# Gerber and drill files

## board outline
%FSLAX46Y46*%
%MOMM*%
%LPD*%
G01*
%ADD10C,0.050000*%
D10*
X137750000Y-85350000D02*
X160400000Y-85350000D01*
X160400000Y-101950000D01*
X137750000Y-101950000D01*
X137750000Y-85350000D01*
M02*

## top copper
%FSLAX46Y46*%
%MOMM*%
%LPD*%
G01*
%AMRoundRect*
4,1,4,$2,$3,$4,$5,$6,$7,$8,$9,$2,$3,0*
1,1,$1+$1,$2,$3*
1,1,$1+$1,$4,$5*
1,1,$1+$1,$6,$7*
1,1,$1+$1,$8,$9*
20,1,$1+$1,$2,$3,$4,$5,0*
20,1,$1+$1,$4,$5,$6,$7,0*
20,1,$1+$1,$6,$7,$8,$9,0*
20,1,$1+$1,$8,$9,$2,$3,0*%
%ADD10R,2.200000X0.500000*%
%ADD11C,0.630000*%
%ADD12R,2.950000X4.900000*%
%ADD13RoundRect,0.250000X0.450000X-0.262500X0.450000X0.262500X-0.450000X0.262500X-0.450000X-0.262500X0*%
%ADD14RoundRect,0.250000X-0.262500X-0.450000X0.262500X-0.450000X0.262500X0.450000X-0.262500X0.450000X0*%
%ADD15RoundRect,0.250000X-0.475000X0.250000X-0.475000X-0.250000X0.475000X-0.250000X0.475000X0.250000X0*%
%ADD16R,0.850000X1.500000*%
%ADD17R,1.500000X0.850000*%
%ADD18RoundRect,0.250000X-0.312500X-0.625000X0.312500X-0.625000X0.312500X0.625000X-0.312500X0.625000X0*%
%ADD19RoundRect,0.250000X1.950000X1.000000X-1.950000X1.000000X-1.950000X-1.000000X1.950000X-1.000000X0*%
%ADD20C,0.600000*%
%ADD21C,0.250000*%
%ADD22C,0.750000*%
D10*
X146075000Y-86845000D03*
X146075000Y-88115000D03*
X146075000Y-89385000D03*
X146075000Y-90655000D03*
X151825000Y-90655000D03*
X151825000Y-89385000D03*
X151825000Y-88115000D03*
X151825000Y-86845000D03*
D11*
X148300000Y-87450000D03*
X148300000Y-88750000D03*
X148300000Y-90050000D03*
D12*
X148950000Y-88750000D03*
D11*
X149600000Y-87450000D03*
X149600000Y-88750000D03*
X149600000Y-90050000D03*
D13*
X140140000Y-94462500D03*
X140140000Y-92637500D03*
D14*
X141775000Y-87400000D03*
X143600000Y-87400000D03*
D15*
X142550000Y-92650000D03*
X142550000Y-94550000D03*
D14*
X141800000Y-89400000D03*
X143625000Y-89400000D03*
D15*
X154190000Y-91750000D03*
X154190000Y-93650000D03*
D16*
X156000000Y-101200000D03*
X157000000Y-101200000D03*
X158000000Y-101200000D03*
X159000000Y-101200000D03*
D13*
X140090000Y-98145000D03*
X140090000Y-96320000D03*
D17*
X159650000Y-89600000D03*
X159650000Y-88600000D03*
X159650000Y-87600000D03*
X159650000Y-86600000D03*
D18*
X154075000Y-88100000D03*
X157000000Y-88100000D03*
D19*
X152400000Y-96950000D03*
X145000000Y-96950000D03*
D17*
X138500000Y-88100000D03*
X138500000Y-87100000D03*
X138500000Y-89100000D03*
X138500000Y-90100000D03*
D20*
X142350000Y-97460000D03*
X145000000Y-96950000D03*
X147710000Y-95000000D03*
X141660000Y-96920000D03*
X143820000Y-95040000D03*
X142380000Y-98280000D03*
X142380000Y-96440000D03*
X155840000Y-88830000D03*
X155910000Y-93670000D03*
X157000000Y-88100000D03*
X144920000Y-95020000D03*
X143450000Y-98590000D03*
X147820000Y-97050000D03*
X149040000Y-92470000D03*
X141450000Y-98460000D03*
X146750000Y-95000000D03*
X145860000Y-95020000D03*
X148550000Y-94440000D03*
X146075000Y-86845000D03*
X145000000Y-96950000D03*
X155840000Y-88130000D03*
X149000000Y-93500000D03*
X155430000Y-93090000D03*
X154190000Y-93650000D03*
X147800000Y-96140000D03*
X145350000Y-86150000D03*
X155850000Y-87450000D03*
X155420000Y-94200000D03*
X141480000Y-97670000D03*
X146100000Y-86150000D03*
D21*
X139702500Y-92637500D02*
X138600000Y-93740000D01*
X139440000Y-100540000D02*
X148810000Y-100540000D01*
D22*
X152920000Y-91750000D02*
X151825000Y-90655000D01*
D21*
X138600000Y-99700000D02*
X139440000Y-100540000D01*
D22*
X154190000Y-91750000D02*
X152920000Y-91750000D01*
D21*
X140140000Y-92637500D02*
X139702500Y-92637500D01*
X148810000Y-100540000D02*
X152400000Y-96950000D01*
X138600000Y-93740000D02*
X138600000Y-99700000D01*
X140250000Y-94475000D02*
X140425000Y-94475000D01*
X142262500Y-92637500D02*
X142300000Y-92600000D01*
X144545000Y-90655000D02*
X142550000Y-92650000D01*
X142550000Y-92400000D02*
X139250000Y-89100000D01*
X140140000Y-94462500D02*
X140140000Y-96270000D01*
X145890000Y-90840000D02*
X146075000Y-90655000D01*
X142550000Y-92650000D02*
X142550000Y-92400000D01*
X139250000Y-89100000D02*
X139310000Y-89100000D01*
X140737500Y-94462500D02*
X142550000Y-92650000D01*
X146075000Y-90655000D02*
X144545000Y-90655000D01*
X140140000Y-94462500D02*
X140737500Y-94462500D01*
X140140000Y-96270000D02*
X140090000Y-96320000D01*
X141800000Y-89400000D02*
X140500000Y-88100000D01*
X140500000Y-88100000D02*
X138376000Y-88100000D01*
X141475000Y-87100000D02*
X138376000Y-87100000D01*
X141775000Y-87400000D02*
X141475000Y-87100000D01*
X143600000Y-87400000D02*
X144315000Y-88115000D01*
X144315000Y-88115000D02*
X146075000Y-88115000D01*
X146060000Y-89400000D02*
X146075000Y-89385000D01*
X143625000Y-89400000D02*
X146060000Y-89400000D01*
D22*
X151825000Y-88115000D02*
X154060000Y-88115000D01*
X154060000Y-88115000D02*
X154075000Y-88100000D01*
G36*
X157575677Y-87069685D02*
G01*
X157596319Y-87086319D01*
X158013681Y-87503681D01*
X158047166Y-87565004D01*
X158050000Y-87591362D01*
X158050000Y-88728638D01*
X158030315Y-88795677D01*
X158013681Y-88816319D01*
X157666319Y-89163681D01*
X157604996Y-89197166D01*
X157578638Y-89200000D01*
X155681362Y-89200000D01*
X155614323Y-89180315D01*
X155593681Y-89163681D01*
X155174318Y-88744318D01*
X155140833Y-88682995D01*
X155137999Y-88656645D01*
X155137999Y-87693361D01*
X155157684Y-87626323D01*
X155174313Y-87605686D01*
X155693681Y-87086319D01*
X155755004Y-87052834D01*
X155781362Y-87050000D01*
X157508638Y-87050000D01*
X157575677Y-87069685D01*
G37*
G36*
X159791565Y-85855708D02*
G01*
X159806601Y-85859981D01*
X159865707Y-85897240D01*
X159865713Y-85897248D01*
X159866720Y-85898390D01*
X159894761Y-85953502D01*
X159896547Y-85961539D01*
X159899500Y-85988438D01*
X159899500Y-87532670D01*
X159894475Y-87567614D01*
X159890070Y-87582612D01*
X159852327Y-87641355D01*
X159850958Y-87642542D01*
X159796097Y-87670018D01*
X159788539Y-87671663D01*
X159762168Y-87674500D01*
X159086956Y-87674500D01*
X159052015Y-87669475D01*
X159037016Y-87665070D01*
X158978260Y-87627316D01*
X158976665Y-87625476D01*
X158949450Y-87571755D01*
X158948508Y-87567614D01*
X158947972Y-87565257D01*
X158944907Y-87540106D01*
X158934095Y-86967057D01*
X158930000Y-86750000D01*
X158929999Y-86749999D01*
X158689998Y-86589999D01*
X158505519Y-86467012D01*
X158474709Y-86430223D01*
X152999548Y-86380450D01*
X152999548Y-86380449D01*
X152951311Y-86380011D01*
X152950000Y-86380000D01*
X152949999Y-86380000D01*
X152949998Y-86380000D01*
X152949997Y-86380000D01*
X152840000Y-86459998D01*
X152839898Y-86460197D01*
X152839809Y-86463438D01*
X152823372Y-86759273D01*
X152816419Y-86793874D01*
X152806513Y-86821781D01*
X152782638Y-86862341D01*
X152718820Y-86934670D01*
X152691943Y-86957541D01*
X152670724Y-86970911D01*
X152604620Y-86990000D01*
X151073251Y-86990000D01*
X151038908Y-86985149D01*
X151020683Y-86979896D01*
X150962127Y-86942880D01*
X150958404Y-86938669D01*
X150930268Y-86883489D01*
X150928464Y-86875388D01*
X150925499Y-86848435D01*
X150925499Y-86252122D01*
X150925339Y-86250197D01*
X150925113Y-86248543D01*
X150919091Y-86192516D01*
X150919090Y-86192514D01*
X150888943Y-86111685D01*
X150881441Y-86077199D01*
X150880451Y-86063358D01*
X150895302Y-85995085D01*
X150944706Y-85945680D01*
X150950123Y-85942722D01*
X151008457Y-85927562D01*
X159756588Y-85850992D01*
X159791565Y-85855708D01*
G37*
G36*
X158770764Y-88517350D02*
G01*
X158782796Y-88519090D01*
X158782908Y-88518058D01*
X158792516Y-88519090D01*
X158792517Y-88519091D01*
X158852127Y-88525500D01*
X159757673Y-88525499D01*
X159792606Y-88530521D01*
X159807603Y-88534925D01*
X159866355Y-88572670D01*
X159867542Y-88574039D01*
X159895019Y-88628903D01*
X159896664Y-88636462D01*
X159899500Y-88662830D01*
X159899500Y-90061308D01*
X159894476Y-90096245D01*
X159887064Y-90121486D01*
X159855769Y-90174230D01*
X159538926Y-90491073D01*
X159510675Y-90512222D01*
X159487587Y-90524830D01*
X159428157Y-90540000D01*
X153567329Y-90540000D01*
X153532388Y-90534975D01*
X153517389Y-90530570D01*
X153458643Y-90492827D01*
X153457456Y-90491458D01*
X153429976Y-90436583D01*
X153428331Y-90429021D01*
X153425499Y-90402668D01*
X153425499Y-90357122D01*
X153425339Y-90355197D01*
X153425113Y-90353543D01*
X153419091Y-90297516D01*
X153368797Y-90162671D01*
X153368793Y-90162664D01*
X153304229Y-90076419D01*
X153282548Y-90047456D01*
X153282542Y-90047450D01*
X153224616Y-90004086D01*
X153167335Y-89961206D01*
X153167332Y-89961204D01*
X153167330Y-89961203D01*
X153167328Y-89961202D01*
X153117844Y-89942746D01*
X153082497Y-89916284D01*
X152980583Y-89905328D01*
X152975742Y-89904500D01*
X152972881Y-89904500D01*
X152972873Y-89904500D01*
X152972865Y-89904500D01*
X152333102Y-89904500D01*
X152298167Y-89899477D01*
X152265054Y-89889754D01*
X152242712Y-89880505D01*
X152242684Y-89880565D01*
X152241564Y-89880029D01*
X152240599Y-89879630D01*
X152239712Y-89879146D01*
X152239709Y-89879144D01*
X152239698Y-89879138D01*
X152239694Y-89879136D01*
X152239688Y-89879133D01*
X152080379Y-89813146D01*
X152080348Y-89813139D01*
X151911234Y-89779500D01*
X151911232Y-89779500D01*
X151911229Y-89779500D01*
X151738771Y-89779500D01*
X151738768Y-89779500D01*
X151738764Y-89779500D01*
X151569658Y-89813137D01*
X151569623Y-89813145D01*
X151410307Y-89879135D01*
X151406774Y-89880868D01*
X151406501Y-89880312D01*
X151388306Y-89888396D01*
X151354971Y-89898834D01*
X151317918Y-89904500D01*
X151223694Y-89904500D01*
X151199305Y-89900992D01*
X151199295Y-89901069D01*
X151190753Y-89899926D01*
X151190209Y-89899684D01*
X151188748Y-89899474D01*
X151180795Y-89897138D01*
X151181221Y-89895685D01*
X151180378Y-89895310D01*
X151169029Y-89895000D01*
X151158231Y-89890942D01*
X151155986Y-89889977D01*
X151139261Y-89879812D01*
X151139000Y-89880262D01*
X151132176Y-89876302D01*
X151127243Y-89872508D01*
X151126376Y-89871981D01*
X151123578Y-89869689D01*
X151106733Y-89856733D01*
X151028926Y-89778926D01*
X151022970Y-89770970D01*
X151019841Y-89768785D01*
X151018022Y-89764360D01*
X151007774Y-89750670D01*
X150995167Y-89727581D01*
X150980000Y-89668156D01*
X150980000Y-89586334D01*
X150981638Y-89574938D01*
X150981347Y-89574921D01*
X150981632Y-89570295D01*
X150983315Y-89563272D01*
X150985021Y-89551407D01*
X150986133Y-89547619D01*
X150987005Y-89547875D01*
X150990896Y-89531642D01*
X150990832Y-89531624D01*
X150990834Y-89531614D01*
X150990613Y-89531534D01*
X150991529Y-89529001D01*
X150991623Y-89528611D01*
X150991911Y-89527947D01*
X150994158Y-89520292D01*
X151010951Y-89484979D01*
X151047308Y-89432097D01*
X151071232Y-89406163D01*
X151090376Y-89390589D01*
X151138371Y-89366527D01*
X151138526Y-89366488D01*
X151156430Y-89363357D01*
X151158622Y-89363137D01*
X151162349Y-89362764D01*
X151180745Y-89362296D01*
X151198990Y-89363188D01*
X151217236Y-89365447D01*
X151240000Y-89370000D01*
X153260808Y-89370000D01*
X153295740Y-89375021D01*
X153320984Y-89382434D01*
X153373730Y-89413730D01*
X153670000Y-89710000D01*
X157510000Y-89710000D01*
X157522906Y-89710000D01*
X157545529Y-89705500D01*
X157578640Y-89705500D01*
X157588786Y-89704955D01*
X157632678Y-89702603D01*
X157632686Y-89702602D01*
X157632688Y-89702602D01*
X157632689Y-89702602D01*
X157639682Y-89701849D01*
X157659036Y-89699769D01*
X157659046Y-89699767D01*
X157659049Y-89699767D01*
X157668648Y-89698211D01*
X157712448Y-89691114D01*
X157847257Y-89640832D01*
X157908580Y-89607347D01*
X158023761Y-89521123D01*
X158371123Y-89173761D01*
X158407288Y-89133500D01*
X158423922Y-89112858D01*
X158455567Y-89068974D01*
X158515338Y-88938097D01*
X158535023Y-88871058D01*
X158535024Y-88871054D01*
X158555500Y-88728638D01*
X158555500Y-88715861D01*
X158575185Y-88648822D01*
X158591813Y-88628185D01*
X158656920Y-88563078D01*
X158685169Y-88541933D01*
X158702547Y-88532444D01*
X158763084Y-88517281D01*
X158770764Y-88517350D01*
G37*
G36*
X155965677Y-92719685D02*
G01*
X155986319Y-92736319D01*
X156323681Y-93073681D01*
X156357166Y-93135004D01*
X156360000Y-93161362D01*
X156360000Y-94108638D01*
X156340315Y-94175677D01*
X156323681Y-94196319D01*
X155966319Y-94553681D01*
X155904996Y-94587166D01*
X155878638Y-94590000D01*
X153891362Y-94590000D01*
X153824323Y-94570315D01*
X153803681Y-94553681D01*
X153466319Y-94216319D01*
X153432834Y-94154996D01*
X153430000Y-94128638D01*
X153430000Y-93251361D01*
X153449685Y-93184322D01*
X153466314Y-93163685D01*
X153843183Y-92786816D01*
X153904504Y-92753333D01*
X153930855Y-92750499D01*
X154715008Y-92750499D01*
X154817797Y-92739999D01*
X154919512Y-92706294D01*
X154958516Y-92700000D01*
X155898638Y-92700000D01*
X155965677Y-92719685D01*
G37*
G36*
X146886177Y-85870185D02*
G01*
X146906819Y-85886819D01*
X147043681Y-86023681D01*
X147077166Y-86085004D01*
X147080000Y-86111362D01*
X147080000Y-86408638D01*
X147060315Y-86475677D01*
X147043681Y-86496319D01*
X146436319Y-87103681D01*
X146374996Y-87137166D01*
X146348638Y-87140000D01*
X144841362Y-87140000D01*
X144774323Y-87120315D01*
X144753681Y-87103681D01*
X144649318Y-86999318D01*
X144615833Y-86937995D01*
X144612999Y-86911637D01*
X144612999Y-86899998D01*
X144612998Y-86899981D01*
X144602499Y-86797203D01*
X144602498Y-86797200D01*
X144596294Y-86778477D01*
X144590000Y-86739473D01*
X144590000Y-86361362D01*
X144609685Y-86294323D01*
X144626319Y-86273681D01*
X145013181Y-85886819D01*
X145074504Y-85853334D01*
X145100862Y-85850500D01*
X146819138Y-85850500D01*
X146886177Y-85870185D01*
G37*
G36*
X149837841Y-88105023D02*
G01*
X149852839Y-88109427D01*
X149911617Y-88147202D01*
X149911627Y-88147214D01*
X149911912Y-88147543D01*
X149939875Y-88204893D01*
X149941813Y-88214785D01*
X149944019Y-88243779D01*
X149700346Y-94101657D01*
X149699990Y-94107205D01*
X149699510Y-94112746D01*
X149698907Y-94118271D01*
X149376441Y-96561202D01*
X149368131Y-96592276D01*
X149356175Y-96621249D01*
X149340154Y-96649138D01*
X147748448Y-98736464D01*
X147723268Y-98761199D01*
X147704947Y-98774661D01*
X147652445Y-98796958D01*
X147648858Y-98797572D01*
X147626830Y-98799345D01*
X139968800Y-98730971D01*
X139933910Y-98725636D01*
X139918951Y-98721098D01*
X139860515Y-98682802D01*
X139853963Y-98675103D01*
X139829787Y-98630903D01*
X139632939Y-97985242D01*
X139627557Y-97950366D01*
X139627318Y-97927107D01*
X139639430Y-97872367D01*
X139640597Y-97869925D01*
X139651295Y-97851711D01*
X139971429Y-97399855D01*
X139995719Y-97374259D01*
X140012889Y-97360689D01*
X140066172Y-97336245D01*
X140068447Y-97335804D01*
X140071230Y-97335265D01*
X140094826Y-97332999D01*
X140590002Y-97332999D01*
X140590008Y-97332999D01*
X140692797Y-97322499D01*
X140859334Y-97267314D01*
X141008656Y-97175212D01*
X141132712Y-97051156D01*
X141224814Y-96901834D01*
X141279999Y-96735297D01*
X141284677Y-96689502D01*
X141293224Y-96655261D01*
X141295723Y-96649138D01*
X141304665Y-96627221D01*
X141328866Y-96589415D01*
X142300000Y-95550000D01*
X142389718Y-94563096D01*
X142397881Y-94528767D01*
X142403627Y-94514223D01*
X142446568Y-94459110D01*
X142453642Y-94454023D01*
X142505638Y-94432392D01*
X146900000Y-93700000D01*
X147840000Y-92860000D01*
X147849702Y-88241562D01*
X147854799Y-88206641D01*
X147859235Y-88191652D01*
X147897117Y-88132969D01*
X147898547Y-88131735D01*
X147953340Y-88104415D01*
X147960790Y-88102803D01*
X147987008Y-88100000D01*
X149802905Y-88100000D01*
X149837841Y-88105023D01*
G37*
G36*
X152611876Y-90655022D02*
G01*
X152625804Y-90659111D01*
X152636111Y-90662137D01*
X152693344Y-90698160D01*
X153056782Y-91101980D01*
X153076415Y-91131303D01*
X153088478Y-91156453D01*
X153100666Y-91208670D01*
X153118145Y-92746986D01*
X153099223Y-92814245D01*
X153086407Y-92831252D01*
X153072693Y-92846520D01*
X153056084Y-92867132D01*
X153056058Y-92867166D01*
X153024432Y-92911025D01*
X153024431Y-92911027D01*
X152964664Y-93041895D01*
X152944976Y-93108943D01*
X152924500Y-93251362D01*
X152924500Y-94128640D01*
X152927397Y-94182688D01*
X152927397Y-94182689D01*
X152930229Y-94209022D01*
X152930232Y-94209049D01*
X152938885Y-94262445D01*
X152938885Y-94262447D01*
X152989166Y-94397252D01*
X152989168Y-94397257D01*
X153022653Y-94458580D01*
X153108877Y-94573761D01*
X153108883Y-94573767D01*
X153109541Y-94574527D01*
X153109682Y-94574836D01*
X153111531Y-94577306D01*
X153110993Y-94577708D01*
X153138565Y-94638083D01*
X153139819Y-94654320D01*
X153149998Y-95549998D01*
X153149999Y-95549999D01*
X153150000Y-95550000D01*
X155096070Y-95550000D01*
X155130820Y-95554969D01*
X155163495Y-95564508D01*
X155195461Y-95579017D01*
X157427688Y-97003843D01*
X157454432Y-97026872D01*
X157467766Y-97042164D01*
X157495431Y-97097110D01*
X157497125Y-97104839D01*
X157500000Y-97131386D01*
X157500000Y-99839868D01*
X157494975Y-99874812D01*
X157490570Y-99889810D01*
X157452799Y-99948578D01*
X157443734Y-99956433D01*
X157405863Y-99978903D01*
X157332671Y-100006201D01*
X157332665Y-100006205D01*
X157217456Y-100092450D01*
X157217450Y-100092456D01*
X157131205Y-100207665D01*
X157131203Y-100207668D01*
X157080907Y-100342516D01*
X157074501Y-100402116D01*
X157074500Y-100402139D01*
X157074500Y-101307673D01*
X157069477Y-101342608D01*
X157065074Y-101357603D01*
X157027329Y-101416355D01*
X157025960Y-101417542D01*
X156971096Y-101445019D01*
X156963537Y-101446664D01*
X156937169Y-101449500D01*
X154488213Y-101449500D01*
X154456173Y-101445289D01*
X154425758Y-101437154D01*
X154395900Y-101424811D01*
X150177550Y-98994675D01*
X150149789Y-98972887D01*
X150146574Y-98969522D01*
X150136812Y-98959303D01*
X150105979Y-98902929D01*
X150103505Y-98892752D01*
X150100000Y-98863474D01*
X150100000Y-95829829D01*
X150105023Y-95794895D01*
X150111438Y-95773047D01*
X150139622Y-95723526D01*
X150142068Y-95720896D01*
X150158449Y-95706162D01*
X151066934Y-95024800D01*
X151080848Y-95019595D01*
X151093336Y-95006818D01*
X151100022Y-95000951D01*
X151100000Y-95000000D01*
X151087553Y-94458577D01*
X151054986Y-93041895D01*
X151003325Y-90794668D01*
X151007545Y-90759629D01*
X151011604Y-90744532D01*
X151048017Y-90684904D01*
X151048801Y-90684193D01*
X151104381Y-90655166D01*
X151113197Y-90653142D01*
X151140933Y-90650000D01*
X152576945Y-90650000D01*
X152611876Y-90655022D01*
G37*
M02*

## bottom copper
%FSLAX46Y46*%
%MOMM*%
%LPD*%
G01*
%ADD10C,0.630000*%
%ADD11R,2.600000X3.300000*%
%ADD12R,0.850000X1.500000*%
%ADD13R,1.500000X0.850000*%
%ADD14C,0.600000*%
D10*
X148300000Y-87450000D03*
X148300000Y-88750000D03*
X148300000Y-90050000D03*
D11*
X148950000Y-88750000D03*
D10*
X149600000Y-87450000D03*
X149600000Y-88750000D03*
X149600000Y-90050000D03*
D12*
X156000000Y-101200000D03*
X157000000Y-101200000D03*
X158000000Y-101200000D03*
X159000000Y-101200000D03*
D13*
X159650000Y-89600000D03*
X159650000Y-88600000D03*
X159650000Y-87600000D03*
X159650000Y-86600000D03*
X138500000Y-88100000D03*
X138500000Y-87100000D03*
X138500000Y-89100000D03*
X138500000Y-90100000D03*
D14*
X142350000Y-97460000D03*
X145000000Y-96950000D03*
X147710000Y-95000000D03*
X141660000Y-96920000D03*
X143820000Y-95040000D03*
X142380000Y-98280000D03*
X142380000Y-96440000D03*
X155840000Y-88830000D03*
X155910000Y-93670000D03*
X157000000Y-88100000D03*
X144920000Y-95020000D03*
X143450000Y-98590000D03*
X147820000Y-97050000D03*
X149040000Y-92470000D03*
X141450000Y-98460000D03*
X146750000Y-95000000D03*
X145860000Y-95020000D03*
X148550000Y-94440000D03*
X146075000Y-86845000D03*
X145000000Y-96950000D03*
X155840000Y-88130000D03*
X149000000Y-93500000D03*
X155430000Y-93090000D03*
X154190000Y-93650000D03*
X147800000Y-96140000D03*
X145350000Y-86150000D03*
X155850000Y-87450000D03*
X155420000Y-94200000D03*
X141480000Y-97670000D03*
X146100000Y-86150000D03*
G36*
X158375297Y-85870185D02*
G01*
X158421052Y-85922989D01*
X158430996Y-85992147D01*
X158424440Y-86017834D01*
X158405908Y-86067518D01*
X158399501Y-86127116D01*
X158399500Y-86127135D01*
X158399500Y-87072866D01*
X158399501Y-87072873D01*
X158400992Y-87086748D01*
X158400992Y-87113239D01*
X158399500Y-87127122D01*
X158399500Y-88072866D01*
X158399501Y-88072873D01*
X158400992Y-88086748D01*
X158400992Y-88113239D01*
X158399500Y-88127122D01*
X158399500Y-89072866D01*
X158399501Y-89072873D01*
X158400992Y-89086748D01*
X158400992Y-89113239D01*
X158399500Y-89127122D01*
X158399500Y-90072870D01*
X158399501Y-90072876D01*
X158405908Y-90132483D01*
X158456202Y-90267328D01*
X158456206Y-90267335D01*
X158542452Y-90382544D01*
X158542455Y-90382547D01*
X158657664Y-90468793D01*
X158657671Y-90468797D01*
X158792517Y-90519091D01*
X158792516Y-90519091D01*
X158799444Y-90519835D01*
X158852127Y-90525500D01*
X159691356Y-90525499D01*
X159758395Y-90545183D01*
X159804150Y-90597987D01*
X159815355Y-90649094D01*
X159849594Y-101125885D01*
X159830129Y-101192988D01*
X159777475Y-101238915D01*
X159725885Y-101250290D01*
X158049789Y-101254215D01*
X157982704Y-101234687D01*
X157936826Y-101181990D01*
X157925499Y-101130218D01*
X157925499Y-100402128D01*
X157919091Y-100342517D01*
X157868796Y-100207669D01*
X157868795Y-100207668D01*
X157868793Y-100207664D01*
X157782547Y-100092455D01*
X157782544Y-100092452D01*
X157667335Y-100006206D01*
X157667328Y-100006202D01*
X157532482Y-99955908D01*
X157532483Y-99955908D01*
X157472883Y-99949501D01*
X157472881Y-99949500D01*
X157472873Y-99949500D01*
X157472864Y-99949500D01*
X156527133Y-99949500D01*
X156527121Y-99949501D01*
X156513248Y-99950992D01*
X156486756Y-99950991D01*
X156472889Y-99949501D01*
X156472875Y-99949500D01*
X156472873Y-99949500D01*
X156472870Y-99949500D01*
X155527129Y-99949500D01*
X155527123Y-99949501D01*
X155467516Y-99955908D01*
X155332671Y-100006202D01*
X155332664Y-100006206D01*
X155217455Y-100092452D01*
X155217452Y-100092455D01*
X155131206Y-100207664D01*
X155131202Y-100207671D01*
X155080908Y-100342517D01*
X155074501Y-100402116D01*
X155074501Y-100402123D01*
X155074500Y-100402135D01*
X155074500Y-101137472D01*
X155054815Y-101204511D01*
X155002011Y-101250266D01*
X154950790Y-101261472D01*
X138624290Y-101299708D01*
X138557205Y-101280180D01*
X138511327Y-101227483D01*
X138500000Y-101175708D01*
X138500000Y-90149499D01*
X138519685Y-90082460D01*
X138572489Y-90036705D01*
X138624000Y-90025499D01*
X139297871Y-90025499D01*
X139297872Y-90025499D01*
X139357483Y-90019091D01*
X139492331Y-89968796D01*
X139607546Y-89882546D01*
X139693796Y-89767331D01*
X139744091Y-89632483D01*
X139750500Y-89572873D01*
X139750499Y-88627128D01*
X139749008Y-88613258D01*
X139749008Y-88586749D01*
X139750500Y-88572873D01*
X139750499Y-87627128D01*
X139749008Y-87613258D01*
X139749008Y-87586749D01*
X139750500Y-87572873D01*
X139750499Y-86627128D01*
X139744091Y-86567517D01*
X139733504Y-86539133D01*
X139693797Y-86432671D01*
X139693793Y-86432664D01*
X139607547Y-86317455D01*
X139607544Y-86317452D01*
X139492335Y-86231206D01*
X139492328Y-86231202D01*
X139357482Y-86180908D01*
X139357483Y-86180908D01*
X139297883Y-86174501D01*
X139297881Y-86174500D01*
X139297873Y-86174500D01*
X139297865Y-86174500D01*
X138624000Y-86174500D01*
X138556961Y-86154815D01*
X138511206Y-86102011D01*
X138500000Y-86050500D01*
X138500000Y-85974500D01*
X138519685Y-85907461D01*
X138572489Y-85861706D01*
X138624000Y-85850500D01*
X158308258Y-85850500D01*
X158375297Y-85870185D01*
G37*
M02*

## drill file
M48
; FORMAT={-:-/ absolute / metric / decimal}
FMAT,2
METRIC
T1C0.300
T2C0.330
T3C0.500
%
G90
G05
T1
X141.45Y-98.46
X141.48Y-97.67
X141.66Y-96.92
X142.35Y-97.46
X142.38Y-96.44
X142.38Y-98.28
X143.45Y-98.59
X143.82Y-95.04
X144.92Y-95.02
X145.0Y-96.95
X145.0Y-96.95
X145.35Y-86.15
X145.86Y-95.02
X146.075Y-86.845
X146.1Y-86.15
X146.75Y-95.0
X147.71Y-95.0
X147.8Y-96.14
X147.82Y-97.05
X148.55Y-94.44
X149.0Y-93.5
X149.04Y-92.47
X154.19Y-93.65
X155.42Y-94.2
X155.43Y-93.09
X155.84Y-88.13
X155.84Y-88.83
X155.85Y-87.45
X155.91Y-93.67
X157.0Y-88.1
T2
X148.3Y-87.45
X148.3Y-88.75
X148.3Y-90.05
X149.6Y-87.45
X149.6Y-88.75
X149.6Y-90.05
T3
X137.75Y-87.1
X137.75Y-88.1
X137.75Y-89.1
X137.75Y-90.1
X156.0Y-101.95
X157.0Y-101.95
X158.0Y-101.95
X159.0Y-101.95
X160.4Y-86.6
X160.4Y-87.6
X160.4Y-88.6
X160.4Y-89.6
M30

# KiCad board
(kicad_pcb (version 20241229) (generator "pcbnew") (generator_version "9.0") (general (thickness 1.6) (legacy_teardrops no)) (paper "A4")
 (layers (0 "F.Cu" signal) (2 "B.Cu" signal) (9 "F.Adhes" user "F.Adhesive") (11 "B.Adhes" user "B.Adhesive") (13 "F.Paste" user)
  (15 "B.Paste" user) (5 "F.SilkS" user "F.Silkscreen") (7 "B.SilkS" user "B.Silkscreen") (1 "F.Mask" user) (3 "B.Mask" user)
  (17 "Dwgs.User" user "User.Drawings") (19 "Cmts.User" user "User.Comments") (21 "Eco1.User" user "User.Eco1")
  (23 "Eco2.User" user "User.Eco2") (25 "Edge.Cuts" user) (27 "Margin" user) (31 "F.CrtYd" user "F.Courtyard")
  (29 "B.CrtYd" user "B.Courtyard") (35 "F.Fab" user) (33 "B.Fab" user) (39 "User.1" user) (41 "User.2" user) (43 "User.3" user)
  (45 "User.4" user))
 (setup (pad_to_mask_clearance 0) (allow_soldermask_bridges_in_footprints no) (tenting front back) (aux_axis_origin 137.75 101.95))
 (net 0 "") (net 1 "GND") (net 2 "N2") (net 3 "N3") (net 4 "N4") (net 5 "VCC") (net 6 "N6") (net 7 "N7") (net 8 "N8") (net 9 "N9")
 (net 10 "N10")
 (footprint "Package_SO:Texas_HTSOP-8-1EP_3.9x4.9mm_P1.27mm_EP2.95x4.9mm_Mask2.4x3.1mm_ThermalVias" (layer "F.Cu") (at 148.95 88.75)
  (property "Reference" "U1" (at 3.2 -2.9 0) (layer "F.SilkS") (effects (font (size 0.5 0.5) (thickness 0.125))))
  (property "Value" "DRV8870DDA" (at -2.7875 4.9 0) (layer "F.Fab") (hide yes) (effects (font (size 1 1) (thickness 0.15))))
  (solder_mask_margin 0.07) (pad "" smd rect (at 0 0) (size 2.4 3.1) (layers "F.Mask"))
  (pad "" smd rect (at 0 0) (size 2.4 3.1) (layers "F.Paste"))
  (pad "1" smd rect (at -2.875 -1.905) (size 2.2 0.5) (layers "F.Cu" "F.Mask" "F.Paste") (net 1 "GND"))
  (pad "2" smd rect (at -2.875 -0.635) (size 2.2 0.5) (layers "F.Cu" "F.Mask" "F.Paste") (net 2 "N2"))
  (pad "3" smd rect (at -2.875 0.635) (size 2.2 0.5) (layers "F.Cu" "F.Mask" "F.Paste") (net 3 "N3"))
  (pad "4" smd rect (at -2.875 1.905) (size 2.2 0.5) (layers "F.Cu" "F.Mask" "F.Paste") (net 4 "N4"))
  (pad "5" smd rect (at 2.875 1.905) (size 2.2 0.5) (layers "F.Cu" "F.Mask" "F.Paste") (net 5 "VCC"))
  (pad "6" smd rect (at 2.875 0.635) (size 2.2 0.5) (layers "F.Cu" "F.Mask" "F.Paste") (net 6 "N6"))
  (pad "7" smd rect (at 2.875 -0.635) (size 2.2 0.5) (layers "F.Cu" "F.Mask" "F.Paste") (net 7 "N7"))
  (pad "8" smd rect (at 2.875 -1.905) (size 2.2 0.5) (layers "F.Cu" "F.Mask" "F.Paste") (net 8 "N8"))
  (pad "9" thru_hole circle (at -0.65 -1.3) (size 0.63 0.63) (drill 0.33) (layers "*.Cu" "*.Mask") (remove_unused_layers no) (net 1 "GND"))
  (pad "9" thru_hole circle (at -0.65 0) (size 0.63 0.63) (drill 0.33) (layers "*.Cu" "*.Mask") (remove_unused_layers no) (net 1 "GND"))
  (pad "9" thru_hole circle (at -0.65 1.3) (size 0.63 0.63) (drill 0.33) (layers "*.Cu" "*.Mask") (remove_unused_layers no) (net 1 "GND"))
  (pad "9" smd rect (at 0 0) (size 2.6 3.3) (layers "B.Cu") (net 1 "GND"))
  (pad "9" smd rect (at 0 0) (size 2.95 4.9) (layers "F.Cu") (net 1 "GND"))
  (pad "9" thru_hole circle (at 0.65 -1.3) (size 0.63 0.63) (drill 0.33) (layers "*.Cu" "*.Mask") (remove_unused_layers no) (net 1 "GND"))
  (pad "9" thru_hole circle (at 0.65 0) (size 0.63 0.63) (drill 0.33) (layers "*.Cu" "*.Mask") (remove_unused_layers no) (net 1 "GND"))
  (pad "9" thru_hole circle (at 0.65 1.3) (size 0.63 0.63) (drill 0.33) (layers "*.Cu" "*.Mask") (remove_unused_layers no) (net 1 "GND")))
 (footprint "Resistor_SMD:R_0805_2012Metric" (layer "F.Cu") (at 140.14 93.55 90)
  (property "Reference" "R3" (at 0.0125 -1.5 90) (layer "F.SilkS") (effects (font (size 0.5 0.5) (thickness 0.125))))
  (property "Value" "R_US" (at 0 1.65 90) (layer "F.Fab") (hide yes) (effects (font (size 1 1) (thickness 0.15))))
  (pad "1" smd roundrect (at -0.9125 0 90) (size 1.025 1.4) (layers "F.Cu" "F.Mask" "F.Paste") (roundrect_rratio 0.243902) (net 4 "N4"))
  (pad "2" smd roundrect (at 0.9125 0 90) (size 1.025 1.4) (layers "F.Cu" "F.Mask" "F.Paste") (roundrect_rratio 0.243902) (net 5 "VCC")))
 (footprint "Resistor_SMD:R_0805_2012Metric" (layer "F.Cu") (at 142.6875 87.4)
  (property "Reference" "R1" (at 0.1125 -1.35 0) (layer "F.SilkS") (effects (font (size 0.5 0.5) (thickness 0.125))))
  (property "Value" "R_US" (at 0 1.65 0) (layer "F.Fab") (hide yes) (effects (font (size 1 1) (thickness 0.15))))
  (pad "1" smd roundrect (at -0.9125 0) (size 1.025 1.4) (layers "F.Cu" "F.Mask" "F.Paste") (roundrect_rratio 0.243902) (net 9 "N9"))
  (pad "2" smd roundrect (at 0.9125 0) (size 1.025 1.4) (layers "F.Cu" "F.Mask" "F.Paste") (roundrect_rratio 0.243902) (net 2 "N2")))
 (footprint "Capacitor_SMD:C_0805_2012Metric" (layer "F.Cu") (at 142.55 93.6 -90)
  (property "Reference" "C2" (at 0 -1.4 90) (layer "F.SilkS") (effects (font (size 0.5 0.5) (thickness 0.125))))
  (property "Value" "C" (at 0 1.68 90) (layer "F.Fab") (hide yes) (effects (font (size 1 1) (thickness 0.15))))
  (pad "1" smd roundrect (at -0.95 0 270) (size 1 1.45) (layers "F.Cu" "F.Mask" "F.Paste") (roundrect_rratio 0.25) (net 4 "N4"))
  (pad "2" smd roundrect (at 0.95 0 270) (size 1 1.45) (layers "F.Cu" "F.Mask" "F.Paste") (roundrect_rratio 0.25) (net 1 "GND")))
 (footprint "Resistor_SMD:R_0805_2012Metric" (layer "F.Cu") (at 142.7125 89.4)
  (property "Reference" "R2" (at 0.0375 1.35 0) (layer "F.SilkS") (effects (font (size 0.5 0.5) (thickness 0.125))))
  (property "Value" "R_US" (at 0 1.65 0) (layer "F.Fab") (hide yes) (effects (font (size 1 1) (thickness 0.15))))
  (pad "1" smd roundrect (at -0.9125 0) (size 1.025 1.4) (layers "F.Cu" "F.Mask" "F.Paste") (roundrect_rratio 0.243902) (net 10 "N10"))
  (pad "2" smd roundrect (at 0.9125 0) (size 1.025 1.4) (layers "F.Cu" "F.Mask" "F.Paste") (roundrect_rratio 0.243902) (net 3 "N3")))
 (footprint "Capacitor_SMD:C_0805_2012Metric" (layer "F.Cu") (at 154.19 92.7 -90)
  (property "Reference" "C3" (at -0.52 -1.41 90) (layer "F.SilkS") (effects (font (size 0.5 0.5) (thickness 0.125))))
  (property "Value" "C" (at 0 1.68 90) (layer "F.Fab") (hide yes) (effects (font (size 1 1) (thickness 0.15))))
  (pad "1" smd roundrect (at -0.95 0 270) (size 1 1.45) (layers "F.Cu" "F.Mask" "F.Paste") (roundrect_rratio 0.25) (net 5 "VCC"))
  (pad "2" smd roundrect (at 0.95 0 270) (size 1 1.45) (layers "F.Cu" "F.Mask" "F.Paste") (roundrect_rratio 0.25) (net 1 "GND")))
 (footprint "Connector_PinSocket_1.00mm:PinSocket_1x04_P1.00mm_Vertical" (layer "F.Cu") (at 156 101.45 90)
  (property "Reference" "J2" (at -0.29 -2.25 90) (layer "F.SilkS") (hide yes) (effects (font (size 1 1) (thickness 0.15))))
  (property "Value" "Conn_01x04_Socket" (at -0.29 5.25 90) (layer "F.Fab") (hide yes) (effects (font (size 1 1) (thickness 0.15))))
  (pad "1" thru_hole rect (at -0.5 0 90) (size 1.5 0.85) (drill 0.5 (offset 0.75 0)) (layers "*.Cu" "*.Mask") (remove_unused_layers no)
   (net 5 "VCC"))
  (pad "2" thru_hole rect (at -0.5 1 90) (size 1.5 0.85) (drill 0.5 (offset 0.75 0)) (layers "*.Cu" "*.Mask") (remove_unused_layers no)
   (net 5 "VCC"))
  (pad "3" thru_hole rect (at -0.5 2 90) (size 1.5 0.85) (drill 0.5 (offset 0.75 0)) (layers "*.Cu" "*.Mask") (remove_unused_layers no)
   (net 1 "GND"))
  (pad "4" thru_hole rect (at -0.5 3 90) (size 1.5 0.85) (drill 0.5 (offset 0.75 0)) (layers "*.Cu" "*.Mask") (remove_unused_layers no)
   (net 1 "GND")))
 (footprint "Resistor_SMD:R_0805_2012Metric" (layer "F.Cu") (at 140.09 97.2325 90)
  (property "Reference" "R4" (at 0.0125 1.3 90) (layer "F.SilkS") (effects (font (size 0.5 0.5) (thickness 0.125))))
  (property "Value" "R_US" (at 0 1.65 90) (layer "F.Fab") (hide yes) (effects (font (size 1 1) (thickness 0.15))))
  (pad "1" smd roundrect (at -0.9125 0 90) (size 1.025 1.4) (layers "F.Cu" "F.Mask" "F.Paste") (roundrect_rratio 0.243902) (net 1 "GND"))
  (pad "2" smd roundrect (at 0.9125 0 90) (size 1.025 1.4) (layers "F.Cu" "F.Mask" "F.Paste") (roundrect_rratio 0.243902) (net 4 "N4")))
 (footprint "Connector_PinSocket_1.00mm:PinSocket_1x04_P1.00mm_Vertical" (layer "F.Cu") (at 160.4 89.6 180)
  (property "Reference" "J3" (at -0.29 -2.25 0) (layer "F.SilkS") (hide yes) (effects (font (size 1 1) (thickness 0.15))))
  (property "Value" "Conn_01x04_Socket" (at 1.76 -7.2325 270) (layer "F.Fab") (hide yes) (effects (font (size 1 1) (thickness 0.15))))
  (pad "1" thru_hole rect (at 0 0 180) (size 1.5 0.85) (drill 0.5 (offset 0.75 0)) (layers "*.Cu" "*.Mask") (remove_unused_layers no)
   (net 6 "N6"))
  (pad "2" thru_hole rect (at 0 1 180) (size 1.5 0.85) (drill 0.5 (offset 0.75 0)) (layers "*.Cu" "*.Mask") (remove_unused_layers no)
   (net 6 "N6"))
  (pad "3" thru_hole rect (at 0 2 180) (size 1.5 0.85) (drill 0.5 (offset 0.75 0)) (layers "*.Cu" "*.Mask") (remove_unused_layers no)
   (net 8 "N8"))
  (pad "4" thru_hole rect (at 0 3 180) (size 1.5 0.85) (drill 0.5 (offset 0.75 0)) (layers "*.Cu" "*.Mask") (remove_unused_layers no)
   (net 8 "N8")))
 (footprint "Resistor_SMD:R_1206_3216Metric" (layer "F.Cu") (at 155.5375 88.1)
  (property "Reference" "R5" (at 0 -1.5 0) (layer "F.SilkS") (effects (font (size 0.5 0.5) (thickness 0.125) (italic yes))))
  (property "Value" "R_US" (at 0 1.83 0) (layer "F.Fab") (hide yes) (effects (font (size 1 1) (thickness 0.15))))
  (pad "1" smd roundrect (at -1.4625 0) (size 1.125 1.75) (layers "F.Cu" "F.Mask" "F.Paste") (roundrect_rratio 0.222222) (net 7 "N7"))
  (pad "2" smd roundrect (at 1.4625 0) (size 1.125 1.75) (layers "F.Cu" "F.Mask" "F.Paste") (roundrect_rratio 0.222222) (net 1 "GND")))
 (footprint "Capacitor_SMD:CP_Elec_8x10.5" (layer "F.Cu") (at 148.7 96.95 180)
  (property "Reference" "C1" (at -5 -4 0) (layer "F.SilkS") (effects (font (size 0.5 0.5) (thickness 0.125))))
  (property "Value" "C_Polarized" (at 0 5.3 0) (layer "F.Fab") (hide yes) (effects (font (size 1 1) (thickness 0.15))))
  (pad "1" smd roundrect (at -3.7 0 180) (size 4.4 2.5) (layers "F.Cu" "F.Mask" "F.Paste") (roundrect_rratio 0.1) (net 5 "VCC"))
  (pad "2" smd roundrect (at 3.7 0 180) (size 4.4 2.5) (layers "F.Cu" "F.Mask" "F.Paste") (roundrect_rratio 0.1) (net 1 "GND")))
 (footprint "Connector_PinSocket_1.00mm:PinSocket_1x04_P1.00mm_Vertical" (layer "F.Cu") (at 138.25 87.1)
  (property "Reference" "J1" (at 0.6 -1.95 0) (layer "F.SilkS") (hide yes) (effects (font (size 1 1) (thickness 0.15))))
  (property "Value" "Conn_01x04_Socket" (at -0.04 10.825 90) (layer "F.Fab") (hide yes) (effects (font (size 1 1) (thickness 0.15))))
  (pad "1" thru_hole rect (at -0.5 1) (size 1.5 0.85) (drill 0.5 (offset 0.75 0)) (layers "*.Cu" "*.Mask" "Eco1.User")
   (remove_unused_layers no) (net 10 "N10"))
  (pad "2" thru_hole rect (at -0.5 0) (size 1.5 0.85) (drill 0.5 (offset 0.75 0)) (layers "*.Cu" "B.Mask") (remove_unused_layers no)
   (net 9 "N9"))
  (pad "3" thru_hole rect (at -0.5 2) (size 1.5 0.85) (drill 0.5 (offset 0.75 0)) (layers "*.Cu" "*.Mask") (remove_unused_layers no)
   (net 4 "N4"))
  (pad "4" thru_hole rect (at -0.5 3) (size 1.5 0.85) (drill 0.5 (offset 0.75 0)) (layers "*.Cu" "*.Mask") (remove_unused_layers no)
   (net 1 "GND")))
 (gr_rect (start 137.75 85.35) (end 160.4 101.95) (stroke (width 0.05) (type default)) (fill no) (layer "Edge.Cuts"))
 (via (at 142.35 97.46) (size 0.6) (drill 0.3) (layers "F.Cu" "B.Cu") (free yes) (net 1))
 (via (at 145 96.95) (size 0.6) (drill 0.3) (layers "F.Cu" "B.Cu") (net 1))
 (via (at 147.71 95) (size 0.6) (drill 0.3) (layers "F.Cu" "B.Cu") (free yes) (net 1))
 (via (at 141.66 96.92) (size 0.6) (drill 0.3) (layers "F.Cu" "B.Cu") (free yes) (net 1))
 (via (at 143.82 95.04) (size 0.6) (drill 0.3) (layers "F.Cu" "B.Cu") (free yes) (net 1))
 (via (at 142.38 98.28) (size 0.6) (drill 0.3) (layers "F.Cu" "B.Cu") (free yes) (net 1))
 (via (at 142.38 96.44) (size 0.6) (drill 0.3) (layers "F.Cu" "B.Cu") (free yes) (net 1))
 (via (at 155.84 88.83) (size 0.6) (drill 0.3) (layers "F.Cu" "B.Cu") (free yes) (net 1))
 (via (at 155.91 93.67) (size 0.6) (drill 0.3) (layers "F.Cu" "B.Cu") (free yes) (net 1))
 (via (at 157 88.1) (size 0.6) (drill 0.3) (layers "F.Cu" "B.Cu") (free yes) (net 1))
 (via (at 144.92 95.02) (size 0.6) (drill 0.3) (layers "F.Cu" "B.Cu") (free yes) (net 1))
 (via (at 143.45 98.59) (size 0.6) (drill 0.3) (layers "F.Cu" "B.Cu") (free yes) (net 1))
 (via (at 147.82 97.05) (size 0.6) (drill 0.3) (layers "F.Cu" "B.Cu") (free yes) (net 1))
 (via (at 149.04 92.47) (size 0.6) (drill 0.3) (layers "F.Cu" "B.Cu") (free yes) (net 1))
 (via (at 141.45 98.46) (size 0.6) (drill 0.3) (layers "F.Cu" "B.Cu") (free yes) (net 1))
 (via (at 146.75 95) (size 0.6) (drill 0.3) (layers "F.Cu" "B.Cu") (free yes) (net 1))
 (via (at 145.86 95.02) (size 0.6) (drill 0.3) (layers "F.Cu" "B.Cu") (free yes) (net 1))
 (via (at 148.55 94.44) (size 0.6) (drill 0.3) (layers "F.Cu" "B.Cu") (free yes) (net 1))
 (via (at 146.075 86.845) (size 0.6) (drill 0.3) (layers "F.Cu" "B.Cu") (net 1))
 (via (at 145 96.95) (size 0.6) (drill 0.3) (layers "F.Cu" "B.Cu") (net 1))
 (via (at 155.84 88.13) (size 0.6) (drill 0.3) (layers "F.Cu" "B.Cu") (free yes) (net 1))
 (via (at 149 93.5) (size 0.6) (drill 0.3) (layers "F.Cu" "B.Cu") (free yes) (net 1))
 (via (at 155.43 93.09) (size 0.6) (drill 0.3) (layers "F.Cu" "B.Cu") (free yes) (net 1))
 (via (at 154.19 93.65) (size 0.6) (drill 0.3) (layers "F.Cu" "B.Cu") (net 1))
 (via (at 147.8 96.14) (size 0.6) (drill 0.3) (layers "F.Cu" "B.Cu") (free yes) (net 1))
 (via (at 145.35 86.15) (size 0.6) (drill 0.3) (layers "F.Cu" "B.Cu") (free yes) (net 1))
 (via (at 155.85 87.45) (size 0.6) (drill 0.3) (layers "F.Cu" "B.Cu") (free yes) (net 1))
 (via (at 155.42 94.2) (size 0.6) (drill 0.3) (layers "F.Cu" "B.Cu") (free yes) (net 1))
 (via (at 141.48 97.67) (size 0.6) (drill 0.3) (layers "F.Cu" "B.Cu") (free yes) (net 1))
 (via (at 146.1 86.15) (size 0.6) (drill 0.3) (layers "F.Cu" "B.Cu") (free yes) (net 1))
 (segment (start 139.7025 92.6375) (end 138.6 93.74) (width 0.25) (layer "F.Cu") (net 5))
 (segment (start 139.44 100.54) (end 148.81 100.54) (width 0.25) (layer "F.Cu") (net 5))
 (segment (start 152.92 91.75) (end 151.825 90.655) (width 0.75) (layer "F.Cu") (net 5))
 (segment (start 138.6 99.7) (end 139.44 100.54) (width 0.25) (layer "F.Cu") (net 5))
 (segment (start 154.19 91.75) (end 152.92 91.75) (width 0.75) (layer "F.Cu") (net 5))
 (segment (start 140.14 92.6375) (end 139.7025 92.6375) (width 0.25) (layer "F.Cu") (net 5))
 (segment (start 148.81 100.54) (end 152.4 96.95) (width 0.25) (layer "F.Cu") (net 5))
 (segment (start 138.6 93.74) (end 138.6 99.7) (width 0.25) (layer "F.Cu") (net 5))
 (segment (start 140.25 94.475) (end 140.425 94.475) (width 0.25) (layer "F.Cu") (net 4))
 (segment (start 142.2625 92.6375) (end 142.3 92.6) (width 0.25) (layer "F.Cu") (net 4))
 (segment (start 144.545 90.655) (end 142.55 92.65) (width 0.25) (layer "F.Cu") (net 4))
 (segment (start 142.55 92.4) (end 139.25 89.1) (width 0.25) (layer "F.Cu") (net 4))
 (segment (start 140.14 94.4625) (end 140.14 96.27) (width 0.25) (layer "F.Cu") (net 4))
 (segment (start 145.89 90.84) (end 146.075 90.655) (width 0.25) (layer "F.Cu") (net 4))
 (segment (start 142.55 92.65) (end 142.55 92.4) (width 0.25) (layer "F.Cu") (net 4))
 (segment (start 139.25 89.1) (end 139.31 89.1) (width 0.25) (layer "F.Cu") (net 4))
 (segment (start 140.7375 94.4625) (end 142.55 92.65) (width 0.25) (layer "F.Cu") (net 4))
 (segment (start 146.075 90.655) (end 144.545 90.655) (width 0.25) (layer "F.Cu") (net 4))
 (segment (start 140.14 94.4625) (end 140.7375 94.4625) (width 0.25) (layer "F.Cu") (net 4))
 (segment (start 140.14 96.27) (end 140.09 96.32) (width 0.25) (layer "F.Cu") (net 4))
 (segment (start 141.8 89.4) (end 140.5 88.1) (width 0.25) (layer "F.Cu") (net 10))
 (segment (start 140.5 88.1) (end 138.376 88.1) (width 0.25) (layer "F.Cu") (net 10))
 (segment (start 141.475 87.1) (end 138.376 87.1) (width 0.25) (layer "F.Cu") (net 9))
 (segment (start 141.775 87.4) (end 141.475 87.1) (width 0.25) (layer "F.Cu") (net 9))
 (segment (start 143.6 87.4) (end 144.315 88.115) (width 0.25) (layer "F.Cu") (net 2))
 (segment (start 144.315 88.115) (end 146.075 88.115) (width 0.25) (layer "F.Cu") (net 2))
 (segment (start 146.06 89.4) (end 146.075 89.385) (width 0.25) (layer "F.Cu") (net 3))
 (segment (start 143.625 89.4) (end 146.06 89.4) (width 0.25) (layer "F.Cu") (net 3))
 (segment (start 151.825 88.115) (end 154.06 88.115) (width 0.75) (layer "F.Cu") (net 7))
 (segment (start 154.06 88.115) (end 154.075 88.1) (width 0.75) (layer "F.Cu") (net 7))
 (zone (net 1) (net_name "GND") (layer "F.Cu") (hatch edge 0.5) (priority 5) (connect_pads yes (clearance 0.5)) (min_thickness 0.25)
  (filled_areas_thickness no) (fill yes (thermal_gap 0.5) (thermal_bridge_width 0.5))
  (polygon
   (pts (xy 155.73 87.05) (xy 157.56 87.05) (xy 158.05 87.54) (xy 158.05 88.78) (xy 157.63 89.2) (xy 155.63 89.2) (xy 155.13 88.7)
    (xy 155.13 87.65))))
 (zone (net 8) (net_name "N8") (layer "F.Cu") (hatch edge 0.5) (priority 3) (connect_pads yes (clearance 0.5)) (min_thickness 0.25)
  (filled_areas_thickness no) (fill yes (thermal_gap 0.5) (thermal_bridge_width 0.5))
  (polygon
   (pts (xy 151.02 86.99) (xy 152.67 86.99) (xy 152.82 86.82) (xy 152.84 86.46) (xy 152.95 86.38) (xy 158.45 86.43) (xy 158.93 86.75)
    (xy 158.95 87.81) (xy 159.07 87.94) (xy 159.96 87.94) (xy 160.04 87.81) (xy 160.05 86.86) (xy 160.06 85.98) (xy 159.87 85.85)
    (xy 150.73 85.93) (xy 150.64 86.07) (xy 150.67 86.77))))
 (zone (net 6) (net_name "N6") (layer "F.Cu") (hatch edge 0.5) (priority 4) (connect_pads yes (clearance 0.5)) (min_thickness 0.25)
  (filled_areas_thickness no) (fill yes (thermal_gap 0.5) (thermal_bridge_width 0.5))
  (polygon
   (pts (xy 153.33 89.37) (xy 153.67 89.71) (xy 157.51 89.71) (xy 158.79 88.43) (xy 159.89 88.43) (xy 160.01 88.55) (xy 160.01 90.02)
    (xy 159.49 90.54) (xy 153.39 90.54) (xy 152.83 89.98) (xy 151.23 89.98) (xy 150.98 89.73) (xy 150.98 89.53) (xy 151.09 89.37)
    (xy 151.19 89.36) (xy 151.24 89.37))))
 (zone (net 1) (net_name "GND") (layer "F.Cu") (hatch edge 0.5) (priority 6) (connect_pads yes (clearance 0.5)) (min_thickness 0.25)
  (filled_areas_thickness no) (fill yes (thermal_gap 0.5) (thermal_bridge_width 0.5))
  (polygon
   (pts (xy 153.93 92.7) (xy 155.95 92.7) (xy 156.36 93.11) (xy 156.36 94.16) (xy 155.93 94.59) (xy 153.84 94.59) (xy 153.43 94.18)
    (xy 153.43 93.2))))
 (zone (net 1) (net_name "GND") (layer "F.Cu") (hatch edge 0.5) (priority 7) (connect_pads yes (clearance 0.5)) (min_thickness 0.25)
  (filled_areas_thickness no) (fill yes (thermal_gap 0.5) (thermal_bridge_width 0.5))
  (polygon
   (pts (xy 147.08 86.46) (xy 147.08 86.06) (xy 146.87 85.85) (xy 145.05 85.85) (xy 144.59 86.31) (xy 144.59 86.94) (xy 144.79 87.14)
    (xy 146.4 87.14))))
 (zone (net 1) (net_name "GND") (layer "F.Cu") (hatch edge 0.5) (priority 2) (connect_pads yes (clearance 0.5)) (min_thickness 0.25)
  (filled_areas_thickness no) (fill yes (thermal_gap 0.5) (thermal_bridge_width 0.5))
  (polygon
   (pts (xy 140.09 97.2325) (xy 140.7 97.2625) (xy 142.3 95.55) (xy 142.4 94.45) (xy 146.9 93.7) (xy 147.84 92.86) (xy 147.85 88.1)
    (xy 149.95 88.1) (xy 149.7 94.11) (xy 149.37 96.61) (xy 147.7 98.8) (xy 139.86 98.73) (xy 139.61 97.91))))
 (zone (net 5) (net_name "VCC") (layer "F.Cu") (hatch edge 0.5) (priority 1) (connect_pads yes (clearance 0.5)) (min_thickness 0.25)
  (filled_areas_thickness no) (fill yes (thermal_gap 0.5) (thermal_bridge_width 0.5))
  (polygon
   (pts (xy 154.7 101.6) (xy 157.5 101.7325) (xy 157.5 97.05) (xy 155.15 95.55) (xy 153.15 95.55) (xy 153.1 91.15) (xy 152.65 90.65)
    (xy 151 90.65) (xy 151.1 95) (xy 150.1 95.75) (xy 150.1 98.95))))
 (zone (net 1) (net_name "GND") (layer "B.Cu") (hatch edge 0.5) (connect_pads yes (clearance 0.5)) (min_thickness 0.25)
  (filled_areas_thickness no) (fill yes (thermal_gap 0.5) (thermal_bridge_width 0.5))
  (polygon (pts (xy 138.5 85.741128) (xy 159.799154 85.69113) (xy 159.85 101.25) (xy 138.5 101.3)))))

